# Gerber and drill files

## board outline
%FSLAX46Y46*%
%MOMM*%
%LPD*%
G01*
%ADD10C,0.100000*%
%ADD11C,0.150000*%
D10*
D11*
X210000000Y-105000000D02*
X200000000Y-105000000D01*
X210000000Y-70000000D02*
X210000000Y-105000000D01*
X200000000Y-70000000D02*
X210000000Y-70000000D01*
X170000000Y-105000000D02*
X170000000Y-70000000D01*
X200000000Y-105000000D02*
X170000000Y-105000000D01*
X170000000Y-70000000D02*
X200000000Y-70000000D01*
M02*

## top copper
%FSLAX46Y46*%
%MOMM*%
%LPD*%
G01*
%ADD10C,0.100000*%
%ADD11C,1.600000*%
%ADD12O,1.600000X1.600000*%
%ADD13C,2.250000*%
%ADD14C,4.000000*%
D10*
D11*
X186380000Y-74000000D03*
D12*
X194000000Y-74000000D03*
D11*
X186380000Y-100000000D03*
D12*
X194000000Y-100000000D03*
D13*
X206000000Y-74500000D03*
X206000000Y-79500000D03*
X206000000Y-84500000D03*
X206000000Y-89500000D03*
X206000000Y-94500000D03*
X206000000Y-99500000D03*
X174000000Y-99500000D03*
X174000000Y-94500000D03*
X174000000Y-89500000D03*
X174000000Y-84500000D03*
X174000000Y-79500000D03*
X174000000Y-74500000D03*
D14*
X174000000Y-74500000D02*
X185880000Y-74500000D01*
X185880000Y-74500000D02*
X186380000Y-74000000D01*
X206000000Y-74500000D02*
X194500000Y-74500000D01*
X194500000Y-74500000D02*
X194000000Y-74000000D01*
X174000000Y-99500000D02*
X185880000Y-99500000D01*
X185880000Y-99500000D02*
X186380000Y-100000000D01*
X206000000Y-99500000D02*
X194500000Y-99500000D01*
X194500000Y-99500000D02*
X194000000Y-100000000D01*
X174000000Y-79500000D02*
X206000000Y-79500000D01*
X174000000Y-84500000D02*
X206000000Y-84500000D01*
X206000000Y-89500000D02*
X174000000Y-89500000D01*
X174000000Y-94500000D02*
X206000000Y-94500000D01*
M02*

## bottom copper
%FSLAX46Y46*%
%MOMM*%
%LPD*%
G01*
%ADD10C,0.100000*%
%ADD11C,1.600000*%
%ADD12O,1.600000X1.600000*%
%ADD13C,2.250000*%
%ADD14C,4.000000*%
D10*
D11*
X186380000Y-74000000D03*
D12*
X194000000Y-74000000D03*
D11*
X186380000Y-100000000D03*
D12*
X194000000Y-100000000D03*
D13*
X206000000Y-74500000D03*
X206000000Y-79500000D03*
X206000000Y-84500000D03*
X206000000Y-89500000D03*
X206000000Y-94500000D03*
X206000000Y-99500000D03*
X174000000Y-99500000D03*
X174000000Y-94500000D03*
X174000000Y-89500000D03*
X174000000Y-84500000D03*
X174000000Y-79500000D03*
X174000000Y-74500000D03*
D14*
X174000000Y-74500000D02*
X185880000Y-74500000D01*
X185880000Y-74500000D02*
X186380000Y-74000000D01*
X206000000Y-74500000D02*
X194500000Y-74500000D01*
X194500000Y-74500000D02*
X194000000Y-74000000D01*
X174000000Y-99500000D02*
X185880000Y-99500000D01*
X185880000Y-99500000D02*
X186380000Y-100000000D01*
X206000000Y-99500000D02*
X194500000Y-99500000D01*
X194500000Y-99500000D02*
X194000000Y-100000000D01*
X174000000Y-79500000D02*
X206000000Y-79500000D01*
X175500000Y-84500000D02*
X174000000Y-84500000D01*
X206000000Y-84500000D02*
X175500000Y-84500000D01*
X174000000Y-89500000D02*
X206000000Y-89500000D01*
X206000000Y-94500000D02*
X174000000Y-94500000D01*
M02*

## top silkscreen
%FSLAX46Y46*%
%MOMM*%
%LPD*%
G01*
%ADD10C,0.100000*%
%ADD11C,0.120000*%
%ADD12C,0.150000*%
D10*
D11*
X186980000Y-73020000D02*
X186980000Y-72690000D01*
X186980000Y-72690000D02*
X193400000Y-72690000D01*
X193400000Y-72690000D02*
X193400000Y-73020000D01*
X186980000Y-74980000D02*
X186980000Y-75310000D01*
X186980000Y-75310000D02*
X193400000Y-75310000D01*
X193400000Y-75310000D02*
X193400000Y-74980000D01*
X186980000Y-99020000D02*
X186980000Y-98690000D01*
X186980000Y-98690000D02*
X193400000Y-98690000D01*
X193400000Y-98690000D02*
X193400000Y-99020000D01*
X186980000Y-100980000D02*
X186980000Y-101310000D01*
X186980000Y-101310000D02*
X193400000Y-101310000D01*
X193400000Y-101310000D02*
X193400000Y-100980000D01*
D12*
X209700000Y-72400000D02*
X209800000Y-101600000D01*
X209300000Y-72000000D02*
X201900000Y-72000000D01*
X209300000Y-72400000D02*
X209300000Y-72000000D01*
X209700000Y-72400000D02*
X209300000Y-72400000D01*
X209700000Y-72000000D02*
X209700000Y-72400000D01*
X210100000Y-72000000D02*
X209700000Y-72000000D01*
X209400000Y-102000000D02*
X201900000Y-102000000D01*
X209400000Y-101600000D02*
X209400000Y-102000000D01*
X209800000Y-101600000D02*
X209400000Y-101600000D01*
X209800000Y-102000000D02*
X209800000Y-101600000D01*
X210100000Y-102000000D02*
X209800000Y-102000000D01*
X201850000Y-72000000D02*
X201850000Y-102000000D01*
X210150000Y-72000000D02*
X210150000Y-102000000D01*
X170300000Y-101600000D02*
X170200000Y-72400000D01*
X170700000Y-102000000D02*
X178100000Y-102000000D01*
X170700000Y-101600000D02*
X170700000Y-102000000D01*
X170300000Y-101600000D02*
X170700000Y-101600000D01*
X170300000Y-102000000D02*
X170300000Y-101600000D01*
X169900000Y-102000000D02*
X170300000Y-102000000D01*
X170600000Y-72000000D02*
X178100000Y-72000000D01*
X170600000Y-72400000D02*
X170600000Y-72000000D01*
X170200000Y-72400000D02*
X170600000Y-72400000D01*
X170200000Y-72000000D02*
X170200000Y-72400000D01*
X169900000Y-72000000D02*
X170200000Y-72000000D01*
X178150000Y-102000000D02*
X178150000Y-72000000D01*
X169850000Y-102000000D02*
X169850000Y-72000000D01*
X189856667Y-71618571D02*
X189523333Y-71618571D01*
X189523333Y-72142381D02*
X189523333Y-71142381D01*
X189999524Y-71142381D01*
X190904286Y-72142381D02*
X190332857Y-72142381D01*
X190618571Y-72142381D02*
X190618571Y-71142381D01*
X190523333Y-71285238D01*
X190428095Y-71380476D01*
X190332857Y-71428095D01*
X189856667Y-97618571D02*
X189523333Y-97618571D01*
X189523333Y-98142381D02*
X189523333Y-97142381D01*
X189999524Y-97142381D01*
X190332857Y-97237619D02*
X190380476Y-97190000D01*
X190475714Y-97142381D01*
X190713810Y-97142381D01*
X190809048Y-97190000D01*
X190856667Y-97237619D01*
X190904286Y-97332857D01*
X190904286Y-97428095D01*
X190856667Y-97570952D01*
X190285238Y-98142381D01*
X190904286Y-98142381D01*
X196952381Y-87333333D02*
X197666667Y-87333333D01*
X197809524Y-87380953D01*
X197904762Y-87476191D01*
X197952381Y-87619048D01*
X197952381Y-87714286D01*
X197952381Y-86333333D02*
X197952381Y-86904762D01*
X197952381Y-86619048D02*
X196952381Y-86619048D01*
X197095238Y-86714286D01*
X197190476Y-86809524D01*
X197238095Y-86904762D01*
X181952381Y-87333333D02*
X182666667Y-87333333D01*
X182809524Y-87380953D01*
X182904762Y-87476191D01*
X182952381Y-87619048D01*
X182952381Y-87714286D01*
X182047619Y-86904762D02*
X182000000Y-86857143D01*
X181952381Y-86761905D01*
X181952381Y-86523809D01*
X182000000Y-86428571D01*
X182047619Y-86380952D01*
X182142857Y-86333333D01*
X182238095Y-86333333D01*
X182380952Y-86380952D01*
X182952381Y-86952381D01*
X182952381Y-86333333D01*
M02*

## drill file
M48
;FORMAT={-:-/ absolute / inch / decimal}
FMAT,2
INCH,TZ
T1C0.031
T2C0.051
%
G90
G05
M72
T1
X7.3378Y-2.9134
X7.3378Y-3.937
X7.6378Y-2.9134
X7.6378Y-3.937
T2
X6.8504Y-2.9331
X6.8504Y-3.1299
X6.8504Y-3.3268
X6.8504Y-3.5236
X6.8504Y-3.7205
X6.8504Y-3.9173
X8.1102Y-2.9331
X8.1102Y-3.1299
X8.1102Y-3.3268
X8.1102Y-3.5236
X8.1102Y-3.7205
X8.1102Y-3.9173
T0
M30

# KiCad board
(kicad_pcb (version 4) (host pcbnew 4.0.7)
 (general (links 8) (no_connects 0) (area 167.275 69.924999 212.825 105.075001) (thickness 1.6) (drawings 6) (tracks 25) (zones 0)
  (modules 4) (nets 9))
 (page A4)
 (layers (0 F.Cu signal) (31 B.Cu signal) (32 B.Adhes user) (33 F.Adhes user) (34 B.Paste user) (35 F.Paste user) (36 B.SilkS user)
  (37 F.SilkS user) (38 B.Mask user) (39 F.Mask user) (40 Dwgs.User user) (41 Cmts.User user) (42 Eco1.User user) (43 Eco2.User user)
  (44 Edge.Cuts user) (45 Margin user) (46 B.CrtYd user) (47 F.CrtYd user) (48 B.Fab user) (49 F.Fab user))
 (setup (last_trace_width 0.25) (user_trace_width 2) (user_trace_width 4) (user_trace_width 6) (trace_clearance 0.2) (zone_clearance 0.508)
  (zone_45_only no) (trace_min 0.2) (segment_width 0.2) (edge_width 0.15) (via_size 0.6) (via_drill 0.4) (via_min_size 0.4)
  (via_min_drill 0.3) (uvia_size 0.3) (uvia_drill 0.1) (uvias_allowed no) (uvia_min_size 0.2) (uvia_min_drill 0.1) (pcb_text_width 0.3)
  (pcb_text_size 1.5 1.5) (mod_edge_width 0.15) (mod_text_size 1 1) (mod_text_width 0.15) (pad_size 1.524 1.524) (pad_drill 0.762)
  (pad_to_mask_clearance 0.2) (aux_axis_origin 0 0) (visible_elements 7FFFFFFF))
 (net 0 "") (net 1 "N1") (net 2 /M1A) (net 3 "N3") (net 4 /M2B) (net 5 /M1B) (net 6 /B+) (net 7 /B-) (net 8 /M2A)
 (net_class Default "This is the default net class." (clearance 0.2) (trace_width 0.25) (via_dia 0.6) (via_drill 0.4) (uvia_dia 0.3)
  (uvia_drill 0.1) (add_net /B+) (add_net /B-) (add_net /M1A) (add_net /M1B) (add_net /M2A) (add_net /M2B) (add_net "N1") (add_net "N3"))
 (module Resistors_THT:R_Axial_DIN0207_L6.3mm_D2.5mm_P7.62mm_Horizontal (layer F.Cu) (at 186.38 74)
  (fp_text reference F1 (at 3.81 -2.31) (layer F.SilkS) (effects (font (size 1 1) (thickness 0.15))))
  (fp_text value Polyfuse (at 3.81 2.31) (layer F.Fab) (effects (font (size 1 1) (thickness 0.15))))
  (fp_line (start 0.6 -0.98) (end 0.6 -1.31) (layer F.SilkS) (width 0.12))
  (fp_line (start 0.6 -1.31) (end 7.02 -1.31) (layer F.SilkS) (width 0.12))
  (fp_line (start 7.02 -1.31) (end 7.02 -0.98) (layer F.SilkS) (width 0.12))
  (fp_line (start 0.6 0.98) (end 0.6 1.31) (layer F.SilkS) (width 0.12))
  (fp_line (start 0.6 1.31) (end 7.02 1.31) (layer F.SilkS) (width 0.12))
  (fp_line (start 7.02 1.31) (end 7.02 0.98) (layer F.SilkS) (width 0.12))
  (pad 1 thru_hole circle (at 0 0) (size 1.6 1.6) (drill 0.8) (layers *.Cu *.Mask) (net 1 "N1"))
  (pad 2 thru_hole oval (at 7.62 0) (size 1.6 1.6) (drill 0.8) (layers *.Cu *.Mask) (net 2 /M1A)))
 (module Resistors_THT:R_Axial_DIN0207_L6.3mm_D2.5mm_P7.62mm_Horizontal (layer F.Cu) (at 186.38 100)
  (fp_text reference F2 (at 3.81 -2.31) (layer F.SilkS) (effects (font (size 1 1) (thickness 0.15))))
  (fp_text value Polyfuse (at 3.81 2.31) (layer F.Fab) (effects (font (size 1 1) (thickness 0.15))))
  (fp_line (start 0.6 -0.98) (end 0.6 -1.31) (layer F.SilkS) (width 0.12))
  (fp_line (start 0.6 -1.31) (end 7.02 -1.31) (layer F.SilkS) (width 0.12))
  (fp_line (start 7.02 -1.31) (end 7.02 -0.98) (layer F.SilkS) (width 0.12))
  (fp_line (start 0.6 0.98) (end 0.6 1.31) (layer F.SilkS) (width 0.12))
  (fp_line (start 0.6 1.31) (end 7.02 1.31) (layer F.SilkS) (width 0.12))
  (fp_line (start 7.02 1.31) (end 7.02 0.98) (layer F.SilkS) (width 0.12))
  (pad 1 thru_hole circle (at 0 0) (size 1.6 1.6) (drill 0.8) (layers *.Cu *.Mask) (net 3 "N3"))
  (pad 2 thru_hole oval (at 7.62 0) (size 1.6 1.6) (drill 0.8) (layers *.Cu *.Mask) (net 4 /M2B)))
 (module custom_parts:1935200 (layer F.Cu) (at 206 87 270)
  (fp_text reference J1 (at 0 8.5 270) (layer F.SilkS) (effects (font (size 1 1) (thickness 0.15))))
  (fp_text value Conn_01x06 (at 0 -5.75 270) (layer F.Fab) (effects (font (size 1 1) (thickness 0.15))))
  (fp_line (start -14.6 -3.7) (end 14.6 -3.8) (layer F.SilkS) (width 0.15))
  (fp_line (start -15 -3.3) (end -15 4.1) (layer F.SilkS) (width 0.15))
  (fp_line (start -14.6 -3.3) (end -15 -3.3) (layer F.SilkS) (width 0.15))
  (fp_line (start -14.6 -3.7) (end -14.6 -3.3) (layer F.SilkS) (width 0.15))
  (fp_line (start -15 -3.7) (end -14.6 -3.7) (layer F.SilkS) (width 0.15))
  (fp_line (start -15 -4.1) (end -15 -3.7) (layer F.SilkS) (width 0.15))
  (fp_line (start 15 -3.4) (end 15 4.1) (layer F.SilkS) (width 0.15))
  (fp_line (start 14.6 -3.4) (end 15 -3.4) (layer F.SilkS) (width 0.15))
  (fp_line (start 14.6 -3.8) (end 14.6 -3.4) (layer F.SilkS) (width 0.15))
  (fp_line (start 15 -3.8) (end 14.6 -3.8) (layer F.SilkS) (width 0.15))
  (fp_line (start 15 -4.1) (end 15 -3.8) (layer F.SilkS) (width 0.15))
  (fp_line (start -15 4.15) (end 15 4.15) (layer F.SilkS) (width 0.15))
  (fp_line (start -15 -4.15) (end 15 -4.15) (layer F.SilkS) (width 0.15))
  (pad 1 thru_hole circle (at -12.5 0 270) (size 2.25 2.25) (drill 1.3) (layers *.Cu *.Mask) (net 2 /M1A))
  (pad 2 thru_hole circle (at -7.5 0 270) (size 2.25 2.25) (drill 1.3) (layers *.Cu *.Mask) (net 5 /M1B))
  (pad 3 thru_hole circle (at -2.5 0 270) (size 2.25 2.25) (drill 1.3) (layers *.Cu *.Mask) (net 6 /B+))
  (pad 4 thru_hole circle (at 2.5 0 270) (size 2.25 2.25) (drill 1.3) (layers *.Cu *.Mask) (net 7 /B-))
  (pad 5 thru_hole circle (at 7.5 0 270) (size 2.25 2.25) (drill 1.3) (layers *.Cu *.Mask) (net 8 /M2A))
  (pad 6 thru_hole circle (at 12.5 0 270) (size 2.25 2.25) (drill 1.3) (layers *.Cu *.Mask) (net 4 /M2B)))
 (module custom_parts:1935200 (layer F.Cu) (at 174 87 90)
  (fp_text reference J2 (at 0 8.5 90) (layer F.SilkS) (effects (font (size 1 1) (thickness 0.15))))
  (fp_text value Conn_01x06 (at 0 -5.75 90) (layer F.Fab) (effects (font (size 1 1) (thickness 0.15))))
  (fp_line (start -14.6 -3.7) (end 14.6 -3.8) (layer F.SilkS) (width 0.15))
  (fp_line (start -15 -3.3) (end -15 4.1) (layer F.SilkS) (width 0.15))
  (fp_line (start -14.6 -3.3) (end -15 -3.3) (layer F.SilkS) (width 0.15))
  (fp_line (start -14.6 -3.7) (end -14.6 -3.3) (layer F.SilkS) (width 0.15))
  (fp_line (start -15 -3.7) (end -14.6 -3.7) (layer F.SilkS) (width 0.15))
  (fp_line (start -15 -4.1) (end -15 -3.7) (layer F.SilkS) (width 0.15))
  (fp_line (start 15 -3.4) (end 15 4.1) (layer F.SilkS) (width 0.15))
  (fp_line (start 14.6 -3.4) (end 15 -3.4) (layer F.SilkS) (width 0.15))
  (fp_line (start 14.6 -3.8) (end 14.6 -3.4) (layer F.SilkS) (width 0.15))
  (fp_line (start 15 -3.8) (end 14.6 -3.8) (layer F.SilkS) (width 0.15))
  (fp_line (start 15 -4.1) (end 15 -3.8) (layer F.SilkS) (width 0.15))
  (fp_line (start -15 4.15) (end 15 4.15) (layer F.SilkS) (width 0.15))
  (fp_line (start -15 -4.15) (end 15 -4.15) (layer F.SilkS) (width 0.15))
  (pad 1 thru_hole circle (at -12.5 0 90) (size 2.25 2.25) (drill 1.3) (layers *.Cu *.Mask) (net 3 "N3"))
  (pad 2 thru_hole circle (at -7.5 0 90) (size 2.25 2.25) (drill 1.3) (layers *.Cu *.Mask) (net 8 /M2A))
  (pad 3 thru_hole circle (at -2.5 0 90) (size 2.25 2.25) (drill 1.3) (layers *.Cu *.Mask) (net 7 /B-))
  (pad 4 thru_hole circle (at 2.5 0 90) (size 2.25 2.25) (drill 1.3) (layers *.Cu *.Mask) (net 6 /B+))
  (pad 5 thru_hole circle (at 7.5 0 90) (size 2.25 2.25) (drill 1.3) (layers *.Cu *.Mask) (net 5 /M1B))
  (pad 6 thru_hole circle (at 12.5 0 90) (size 2.25 2.25) (drill 1.3) (layers *.Cu *.Mask) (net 1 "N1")))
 (gr_line (start 210 105) (end 200 105) (layer Edge.Cuts) (width 0.15))
 (gr_line (start 210 70) (end 210 105) (layer Edge.Cuts) (width 0.15))
 (gr_line (start 200 70) (end 210 70) (layer Edge.Cuts) (width 0.15))
 (gr_line (start 170 105) (end 170 70) (layer Edge.Cuts) (width 0.15))
 (gr_line (start 200 105) (end 170 105) (layer Edge.Cuts) (width 0.15))
 (gr_line (start 170 70) (end 200 70) (layer Edge.Cuts) (width 0.15))
 (segment (start 174 74.5) (end 185.88 74.5) (width 4) (layer B.Cu) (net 1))
 (segment (start 185.88 74.5) (end 186.38 74) (width 4) (layer B.Cu) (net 1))
 (segment (start 174 74.5) (end 185.88 74.5) (width 4) (layer F.Cu) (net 1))
 (segment (start 185.88 74.5) (end 186.38 74) (width 4) (layer F.Cu) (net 1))
 (segment (start 206 74.5) (end 194.5 74.5) (width 4) (layer B.Cu) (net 2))
 (segment (start 194.5 74.5) (end 194 74) (width 4) (layer B.Cu) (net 2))
 (segment (start 206 74.5) (end 194.5 74.5) (width 4) (layer F.Cu) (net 2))
 (segment (start 194.5 74.5) (end 194 74) (width 4) (layer F.Cu) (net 2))
 (segment (start 174 99.5) (end 185.88 99.5) (width 4) (layer B.Cu) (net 3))
 (segment (start 185.88 99.5) (end 186.38 100) (width 4) (layer B.Cu) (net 3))
 (segment (start 174 99.5) (end 185.88 99.5) (width 4) (layer F.Cu) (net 3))
 (segment (start 185.88 99.5) (end 186.38 100) (width 4) (layer F.Cu) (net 3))
 (segment (start 206 99.5) (end 194.5 99.5) (width 4) (layer B.Cu) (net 4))
 (segment (start 194.5 99.5) (end 194 100) (width 4) (layer B.Cu) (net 4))
 (segment (start 206 99.5) (end 194.5 99.5) (width 4) (layer F.Cu) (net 4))
 (segment (start 194.5 99.5) (end 194 100) (width 4) (layer F.Cu) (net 4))
 (segment (start 174 79.5) (end 206 79.5) (width 4) (layer B.Cu) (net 5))
 (segment (start 174 79.5) (end 206 79.5) (width 4) (layer F.Cu) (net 5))
 (segment (start 175.5 84.5) (end 174 84.5) (width 4) (layer B.Cu) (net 6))
 (segment (start 206 84.5) (end 175.5 84.5) (width 4) (layer B.Cu) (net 6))
 (segment (start 174 84.5) (end 206 84.5) (width 4) (layer F.Cu) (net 6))
 (segment (start 174 89.5) (end 206 89.5) (width 4) (layer B.Cu) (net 7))
 (segment (start 206 89.5) (end 174 89.5) (width 4) (layer F.Cu) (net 7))
 (segment (start 206 94.5) (end 174 94.5) (width 4) (layer B.Cu) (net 8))
 (segment (start 174 94.5) (end 206 94.5) (width 4) (layer F.Cu) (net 8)))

